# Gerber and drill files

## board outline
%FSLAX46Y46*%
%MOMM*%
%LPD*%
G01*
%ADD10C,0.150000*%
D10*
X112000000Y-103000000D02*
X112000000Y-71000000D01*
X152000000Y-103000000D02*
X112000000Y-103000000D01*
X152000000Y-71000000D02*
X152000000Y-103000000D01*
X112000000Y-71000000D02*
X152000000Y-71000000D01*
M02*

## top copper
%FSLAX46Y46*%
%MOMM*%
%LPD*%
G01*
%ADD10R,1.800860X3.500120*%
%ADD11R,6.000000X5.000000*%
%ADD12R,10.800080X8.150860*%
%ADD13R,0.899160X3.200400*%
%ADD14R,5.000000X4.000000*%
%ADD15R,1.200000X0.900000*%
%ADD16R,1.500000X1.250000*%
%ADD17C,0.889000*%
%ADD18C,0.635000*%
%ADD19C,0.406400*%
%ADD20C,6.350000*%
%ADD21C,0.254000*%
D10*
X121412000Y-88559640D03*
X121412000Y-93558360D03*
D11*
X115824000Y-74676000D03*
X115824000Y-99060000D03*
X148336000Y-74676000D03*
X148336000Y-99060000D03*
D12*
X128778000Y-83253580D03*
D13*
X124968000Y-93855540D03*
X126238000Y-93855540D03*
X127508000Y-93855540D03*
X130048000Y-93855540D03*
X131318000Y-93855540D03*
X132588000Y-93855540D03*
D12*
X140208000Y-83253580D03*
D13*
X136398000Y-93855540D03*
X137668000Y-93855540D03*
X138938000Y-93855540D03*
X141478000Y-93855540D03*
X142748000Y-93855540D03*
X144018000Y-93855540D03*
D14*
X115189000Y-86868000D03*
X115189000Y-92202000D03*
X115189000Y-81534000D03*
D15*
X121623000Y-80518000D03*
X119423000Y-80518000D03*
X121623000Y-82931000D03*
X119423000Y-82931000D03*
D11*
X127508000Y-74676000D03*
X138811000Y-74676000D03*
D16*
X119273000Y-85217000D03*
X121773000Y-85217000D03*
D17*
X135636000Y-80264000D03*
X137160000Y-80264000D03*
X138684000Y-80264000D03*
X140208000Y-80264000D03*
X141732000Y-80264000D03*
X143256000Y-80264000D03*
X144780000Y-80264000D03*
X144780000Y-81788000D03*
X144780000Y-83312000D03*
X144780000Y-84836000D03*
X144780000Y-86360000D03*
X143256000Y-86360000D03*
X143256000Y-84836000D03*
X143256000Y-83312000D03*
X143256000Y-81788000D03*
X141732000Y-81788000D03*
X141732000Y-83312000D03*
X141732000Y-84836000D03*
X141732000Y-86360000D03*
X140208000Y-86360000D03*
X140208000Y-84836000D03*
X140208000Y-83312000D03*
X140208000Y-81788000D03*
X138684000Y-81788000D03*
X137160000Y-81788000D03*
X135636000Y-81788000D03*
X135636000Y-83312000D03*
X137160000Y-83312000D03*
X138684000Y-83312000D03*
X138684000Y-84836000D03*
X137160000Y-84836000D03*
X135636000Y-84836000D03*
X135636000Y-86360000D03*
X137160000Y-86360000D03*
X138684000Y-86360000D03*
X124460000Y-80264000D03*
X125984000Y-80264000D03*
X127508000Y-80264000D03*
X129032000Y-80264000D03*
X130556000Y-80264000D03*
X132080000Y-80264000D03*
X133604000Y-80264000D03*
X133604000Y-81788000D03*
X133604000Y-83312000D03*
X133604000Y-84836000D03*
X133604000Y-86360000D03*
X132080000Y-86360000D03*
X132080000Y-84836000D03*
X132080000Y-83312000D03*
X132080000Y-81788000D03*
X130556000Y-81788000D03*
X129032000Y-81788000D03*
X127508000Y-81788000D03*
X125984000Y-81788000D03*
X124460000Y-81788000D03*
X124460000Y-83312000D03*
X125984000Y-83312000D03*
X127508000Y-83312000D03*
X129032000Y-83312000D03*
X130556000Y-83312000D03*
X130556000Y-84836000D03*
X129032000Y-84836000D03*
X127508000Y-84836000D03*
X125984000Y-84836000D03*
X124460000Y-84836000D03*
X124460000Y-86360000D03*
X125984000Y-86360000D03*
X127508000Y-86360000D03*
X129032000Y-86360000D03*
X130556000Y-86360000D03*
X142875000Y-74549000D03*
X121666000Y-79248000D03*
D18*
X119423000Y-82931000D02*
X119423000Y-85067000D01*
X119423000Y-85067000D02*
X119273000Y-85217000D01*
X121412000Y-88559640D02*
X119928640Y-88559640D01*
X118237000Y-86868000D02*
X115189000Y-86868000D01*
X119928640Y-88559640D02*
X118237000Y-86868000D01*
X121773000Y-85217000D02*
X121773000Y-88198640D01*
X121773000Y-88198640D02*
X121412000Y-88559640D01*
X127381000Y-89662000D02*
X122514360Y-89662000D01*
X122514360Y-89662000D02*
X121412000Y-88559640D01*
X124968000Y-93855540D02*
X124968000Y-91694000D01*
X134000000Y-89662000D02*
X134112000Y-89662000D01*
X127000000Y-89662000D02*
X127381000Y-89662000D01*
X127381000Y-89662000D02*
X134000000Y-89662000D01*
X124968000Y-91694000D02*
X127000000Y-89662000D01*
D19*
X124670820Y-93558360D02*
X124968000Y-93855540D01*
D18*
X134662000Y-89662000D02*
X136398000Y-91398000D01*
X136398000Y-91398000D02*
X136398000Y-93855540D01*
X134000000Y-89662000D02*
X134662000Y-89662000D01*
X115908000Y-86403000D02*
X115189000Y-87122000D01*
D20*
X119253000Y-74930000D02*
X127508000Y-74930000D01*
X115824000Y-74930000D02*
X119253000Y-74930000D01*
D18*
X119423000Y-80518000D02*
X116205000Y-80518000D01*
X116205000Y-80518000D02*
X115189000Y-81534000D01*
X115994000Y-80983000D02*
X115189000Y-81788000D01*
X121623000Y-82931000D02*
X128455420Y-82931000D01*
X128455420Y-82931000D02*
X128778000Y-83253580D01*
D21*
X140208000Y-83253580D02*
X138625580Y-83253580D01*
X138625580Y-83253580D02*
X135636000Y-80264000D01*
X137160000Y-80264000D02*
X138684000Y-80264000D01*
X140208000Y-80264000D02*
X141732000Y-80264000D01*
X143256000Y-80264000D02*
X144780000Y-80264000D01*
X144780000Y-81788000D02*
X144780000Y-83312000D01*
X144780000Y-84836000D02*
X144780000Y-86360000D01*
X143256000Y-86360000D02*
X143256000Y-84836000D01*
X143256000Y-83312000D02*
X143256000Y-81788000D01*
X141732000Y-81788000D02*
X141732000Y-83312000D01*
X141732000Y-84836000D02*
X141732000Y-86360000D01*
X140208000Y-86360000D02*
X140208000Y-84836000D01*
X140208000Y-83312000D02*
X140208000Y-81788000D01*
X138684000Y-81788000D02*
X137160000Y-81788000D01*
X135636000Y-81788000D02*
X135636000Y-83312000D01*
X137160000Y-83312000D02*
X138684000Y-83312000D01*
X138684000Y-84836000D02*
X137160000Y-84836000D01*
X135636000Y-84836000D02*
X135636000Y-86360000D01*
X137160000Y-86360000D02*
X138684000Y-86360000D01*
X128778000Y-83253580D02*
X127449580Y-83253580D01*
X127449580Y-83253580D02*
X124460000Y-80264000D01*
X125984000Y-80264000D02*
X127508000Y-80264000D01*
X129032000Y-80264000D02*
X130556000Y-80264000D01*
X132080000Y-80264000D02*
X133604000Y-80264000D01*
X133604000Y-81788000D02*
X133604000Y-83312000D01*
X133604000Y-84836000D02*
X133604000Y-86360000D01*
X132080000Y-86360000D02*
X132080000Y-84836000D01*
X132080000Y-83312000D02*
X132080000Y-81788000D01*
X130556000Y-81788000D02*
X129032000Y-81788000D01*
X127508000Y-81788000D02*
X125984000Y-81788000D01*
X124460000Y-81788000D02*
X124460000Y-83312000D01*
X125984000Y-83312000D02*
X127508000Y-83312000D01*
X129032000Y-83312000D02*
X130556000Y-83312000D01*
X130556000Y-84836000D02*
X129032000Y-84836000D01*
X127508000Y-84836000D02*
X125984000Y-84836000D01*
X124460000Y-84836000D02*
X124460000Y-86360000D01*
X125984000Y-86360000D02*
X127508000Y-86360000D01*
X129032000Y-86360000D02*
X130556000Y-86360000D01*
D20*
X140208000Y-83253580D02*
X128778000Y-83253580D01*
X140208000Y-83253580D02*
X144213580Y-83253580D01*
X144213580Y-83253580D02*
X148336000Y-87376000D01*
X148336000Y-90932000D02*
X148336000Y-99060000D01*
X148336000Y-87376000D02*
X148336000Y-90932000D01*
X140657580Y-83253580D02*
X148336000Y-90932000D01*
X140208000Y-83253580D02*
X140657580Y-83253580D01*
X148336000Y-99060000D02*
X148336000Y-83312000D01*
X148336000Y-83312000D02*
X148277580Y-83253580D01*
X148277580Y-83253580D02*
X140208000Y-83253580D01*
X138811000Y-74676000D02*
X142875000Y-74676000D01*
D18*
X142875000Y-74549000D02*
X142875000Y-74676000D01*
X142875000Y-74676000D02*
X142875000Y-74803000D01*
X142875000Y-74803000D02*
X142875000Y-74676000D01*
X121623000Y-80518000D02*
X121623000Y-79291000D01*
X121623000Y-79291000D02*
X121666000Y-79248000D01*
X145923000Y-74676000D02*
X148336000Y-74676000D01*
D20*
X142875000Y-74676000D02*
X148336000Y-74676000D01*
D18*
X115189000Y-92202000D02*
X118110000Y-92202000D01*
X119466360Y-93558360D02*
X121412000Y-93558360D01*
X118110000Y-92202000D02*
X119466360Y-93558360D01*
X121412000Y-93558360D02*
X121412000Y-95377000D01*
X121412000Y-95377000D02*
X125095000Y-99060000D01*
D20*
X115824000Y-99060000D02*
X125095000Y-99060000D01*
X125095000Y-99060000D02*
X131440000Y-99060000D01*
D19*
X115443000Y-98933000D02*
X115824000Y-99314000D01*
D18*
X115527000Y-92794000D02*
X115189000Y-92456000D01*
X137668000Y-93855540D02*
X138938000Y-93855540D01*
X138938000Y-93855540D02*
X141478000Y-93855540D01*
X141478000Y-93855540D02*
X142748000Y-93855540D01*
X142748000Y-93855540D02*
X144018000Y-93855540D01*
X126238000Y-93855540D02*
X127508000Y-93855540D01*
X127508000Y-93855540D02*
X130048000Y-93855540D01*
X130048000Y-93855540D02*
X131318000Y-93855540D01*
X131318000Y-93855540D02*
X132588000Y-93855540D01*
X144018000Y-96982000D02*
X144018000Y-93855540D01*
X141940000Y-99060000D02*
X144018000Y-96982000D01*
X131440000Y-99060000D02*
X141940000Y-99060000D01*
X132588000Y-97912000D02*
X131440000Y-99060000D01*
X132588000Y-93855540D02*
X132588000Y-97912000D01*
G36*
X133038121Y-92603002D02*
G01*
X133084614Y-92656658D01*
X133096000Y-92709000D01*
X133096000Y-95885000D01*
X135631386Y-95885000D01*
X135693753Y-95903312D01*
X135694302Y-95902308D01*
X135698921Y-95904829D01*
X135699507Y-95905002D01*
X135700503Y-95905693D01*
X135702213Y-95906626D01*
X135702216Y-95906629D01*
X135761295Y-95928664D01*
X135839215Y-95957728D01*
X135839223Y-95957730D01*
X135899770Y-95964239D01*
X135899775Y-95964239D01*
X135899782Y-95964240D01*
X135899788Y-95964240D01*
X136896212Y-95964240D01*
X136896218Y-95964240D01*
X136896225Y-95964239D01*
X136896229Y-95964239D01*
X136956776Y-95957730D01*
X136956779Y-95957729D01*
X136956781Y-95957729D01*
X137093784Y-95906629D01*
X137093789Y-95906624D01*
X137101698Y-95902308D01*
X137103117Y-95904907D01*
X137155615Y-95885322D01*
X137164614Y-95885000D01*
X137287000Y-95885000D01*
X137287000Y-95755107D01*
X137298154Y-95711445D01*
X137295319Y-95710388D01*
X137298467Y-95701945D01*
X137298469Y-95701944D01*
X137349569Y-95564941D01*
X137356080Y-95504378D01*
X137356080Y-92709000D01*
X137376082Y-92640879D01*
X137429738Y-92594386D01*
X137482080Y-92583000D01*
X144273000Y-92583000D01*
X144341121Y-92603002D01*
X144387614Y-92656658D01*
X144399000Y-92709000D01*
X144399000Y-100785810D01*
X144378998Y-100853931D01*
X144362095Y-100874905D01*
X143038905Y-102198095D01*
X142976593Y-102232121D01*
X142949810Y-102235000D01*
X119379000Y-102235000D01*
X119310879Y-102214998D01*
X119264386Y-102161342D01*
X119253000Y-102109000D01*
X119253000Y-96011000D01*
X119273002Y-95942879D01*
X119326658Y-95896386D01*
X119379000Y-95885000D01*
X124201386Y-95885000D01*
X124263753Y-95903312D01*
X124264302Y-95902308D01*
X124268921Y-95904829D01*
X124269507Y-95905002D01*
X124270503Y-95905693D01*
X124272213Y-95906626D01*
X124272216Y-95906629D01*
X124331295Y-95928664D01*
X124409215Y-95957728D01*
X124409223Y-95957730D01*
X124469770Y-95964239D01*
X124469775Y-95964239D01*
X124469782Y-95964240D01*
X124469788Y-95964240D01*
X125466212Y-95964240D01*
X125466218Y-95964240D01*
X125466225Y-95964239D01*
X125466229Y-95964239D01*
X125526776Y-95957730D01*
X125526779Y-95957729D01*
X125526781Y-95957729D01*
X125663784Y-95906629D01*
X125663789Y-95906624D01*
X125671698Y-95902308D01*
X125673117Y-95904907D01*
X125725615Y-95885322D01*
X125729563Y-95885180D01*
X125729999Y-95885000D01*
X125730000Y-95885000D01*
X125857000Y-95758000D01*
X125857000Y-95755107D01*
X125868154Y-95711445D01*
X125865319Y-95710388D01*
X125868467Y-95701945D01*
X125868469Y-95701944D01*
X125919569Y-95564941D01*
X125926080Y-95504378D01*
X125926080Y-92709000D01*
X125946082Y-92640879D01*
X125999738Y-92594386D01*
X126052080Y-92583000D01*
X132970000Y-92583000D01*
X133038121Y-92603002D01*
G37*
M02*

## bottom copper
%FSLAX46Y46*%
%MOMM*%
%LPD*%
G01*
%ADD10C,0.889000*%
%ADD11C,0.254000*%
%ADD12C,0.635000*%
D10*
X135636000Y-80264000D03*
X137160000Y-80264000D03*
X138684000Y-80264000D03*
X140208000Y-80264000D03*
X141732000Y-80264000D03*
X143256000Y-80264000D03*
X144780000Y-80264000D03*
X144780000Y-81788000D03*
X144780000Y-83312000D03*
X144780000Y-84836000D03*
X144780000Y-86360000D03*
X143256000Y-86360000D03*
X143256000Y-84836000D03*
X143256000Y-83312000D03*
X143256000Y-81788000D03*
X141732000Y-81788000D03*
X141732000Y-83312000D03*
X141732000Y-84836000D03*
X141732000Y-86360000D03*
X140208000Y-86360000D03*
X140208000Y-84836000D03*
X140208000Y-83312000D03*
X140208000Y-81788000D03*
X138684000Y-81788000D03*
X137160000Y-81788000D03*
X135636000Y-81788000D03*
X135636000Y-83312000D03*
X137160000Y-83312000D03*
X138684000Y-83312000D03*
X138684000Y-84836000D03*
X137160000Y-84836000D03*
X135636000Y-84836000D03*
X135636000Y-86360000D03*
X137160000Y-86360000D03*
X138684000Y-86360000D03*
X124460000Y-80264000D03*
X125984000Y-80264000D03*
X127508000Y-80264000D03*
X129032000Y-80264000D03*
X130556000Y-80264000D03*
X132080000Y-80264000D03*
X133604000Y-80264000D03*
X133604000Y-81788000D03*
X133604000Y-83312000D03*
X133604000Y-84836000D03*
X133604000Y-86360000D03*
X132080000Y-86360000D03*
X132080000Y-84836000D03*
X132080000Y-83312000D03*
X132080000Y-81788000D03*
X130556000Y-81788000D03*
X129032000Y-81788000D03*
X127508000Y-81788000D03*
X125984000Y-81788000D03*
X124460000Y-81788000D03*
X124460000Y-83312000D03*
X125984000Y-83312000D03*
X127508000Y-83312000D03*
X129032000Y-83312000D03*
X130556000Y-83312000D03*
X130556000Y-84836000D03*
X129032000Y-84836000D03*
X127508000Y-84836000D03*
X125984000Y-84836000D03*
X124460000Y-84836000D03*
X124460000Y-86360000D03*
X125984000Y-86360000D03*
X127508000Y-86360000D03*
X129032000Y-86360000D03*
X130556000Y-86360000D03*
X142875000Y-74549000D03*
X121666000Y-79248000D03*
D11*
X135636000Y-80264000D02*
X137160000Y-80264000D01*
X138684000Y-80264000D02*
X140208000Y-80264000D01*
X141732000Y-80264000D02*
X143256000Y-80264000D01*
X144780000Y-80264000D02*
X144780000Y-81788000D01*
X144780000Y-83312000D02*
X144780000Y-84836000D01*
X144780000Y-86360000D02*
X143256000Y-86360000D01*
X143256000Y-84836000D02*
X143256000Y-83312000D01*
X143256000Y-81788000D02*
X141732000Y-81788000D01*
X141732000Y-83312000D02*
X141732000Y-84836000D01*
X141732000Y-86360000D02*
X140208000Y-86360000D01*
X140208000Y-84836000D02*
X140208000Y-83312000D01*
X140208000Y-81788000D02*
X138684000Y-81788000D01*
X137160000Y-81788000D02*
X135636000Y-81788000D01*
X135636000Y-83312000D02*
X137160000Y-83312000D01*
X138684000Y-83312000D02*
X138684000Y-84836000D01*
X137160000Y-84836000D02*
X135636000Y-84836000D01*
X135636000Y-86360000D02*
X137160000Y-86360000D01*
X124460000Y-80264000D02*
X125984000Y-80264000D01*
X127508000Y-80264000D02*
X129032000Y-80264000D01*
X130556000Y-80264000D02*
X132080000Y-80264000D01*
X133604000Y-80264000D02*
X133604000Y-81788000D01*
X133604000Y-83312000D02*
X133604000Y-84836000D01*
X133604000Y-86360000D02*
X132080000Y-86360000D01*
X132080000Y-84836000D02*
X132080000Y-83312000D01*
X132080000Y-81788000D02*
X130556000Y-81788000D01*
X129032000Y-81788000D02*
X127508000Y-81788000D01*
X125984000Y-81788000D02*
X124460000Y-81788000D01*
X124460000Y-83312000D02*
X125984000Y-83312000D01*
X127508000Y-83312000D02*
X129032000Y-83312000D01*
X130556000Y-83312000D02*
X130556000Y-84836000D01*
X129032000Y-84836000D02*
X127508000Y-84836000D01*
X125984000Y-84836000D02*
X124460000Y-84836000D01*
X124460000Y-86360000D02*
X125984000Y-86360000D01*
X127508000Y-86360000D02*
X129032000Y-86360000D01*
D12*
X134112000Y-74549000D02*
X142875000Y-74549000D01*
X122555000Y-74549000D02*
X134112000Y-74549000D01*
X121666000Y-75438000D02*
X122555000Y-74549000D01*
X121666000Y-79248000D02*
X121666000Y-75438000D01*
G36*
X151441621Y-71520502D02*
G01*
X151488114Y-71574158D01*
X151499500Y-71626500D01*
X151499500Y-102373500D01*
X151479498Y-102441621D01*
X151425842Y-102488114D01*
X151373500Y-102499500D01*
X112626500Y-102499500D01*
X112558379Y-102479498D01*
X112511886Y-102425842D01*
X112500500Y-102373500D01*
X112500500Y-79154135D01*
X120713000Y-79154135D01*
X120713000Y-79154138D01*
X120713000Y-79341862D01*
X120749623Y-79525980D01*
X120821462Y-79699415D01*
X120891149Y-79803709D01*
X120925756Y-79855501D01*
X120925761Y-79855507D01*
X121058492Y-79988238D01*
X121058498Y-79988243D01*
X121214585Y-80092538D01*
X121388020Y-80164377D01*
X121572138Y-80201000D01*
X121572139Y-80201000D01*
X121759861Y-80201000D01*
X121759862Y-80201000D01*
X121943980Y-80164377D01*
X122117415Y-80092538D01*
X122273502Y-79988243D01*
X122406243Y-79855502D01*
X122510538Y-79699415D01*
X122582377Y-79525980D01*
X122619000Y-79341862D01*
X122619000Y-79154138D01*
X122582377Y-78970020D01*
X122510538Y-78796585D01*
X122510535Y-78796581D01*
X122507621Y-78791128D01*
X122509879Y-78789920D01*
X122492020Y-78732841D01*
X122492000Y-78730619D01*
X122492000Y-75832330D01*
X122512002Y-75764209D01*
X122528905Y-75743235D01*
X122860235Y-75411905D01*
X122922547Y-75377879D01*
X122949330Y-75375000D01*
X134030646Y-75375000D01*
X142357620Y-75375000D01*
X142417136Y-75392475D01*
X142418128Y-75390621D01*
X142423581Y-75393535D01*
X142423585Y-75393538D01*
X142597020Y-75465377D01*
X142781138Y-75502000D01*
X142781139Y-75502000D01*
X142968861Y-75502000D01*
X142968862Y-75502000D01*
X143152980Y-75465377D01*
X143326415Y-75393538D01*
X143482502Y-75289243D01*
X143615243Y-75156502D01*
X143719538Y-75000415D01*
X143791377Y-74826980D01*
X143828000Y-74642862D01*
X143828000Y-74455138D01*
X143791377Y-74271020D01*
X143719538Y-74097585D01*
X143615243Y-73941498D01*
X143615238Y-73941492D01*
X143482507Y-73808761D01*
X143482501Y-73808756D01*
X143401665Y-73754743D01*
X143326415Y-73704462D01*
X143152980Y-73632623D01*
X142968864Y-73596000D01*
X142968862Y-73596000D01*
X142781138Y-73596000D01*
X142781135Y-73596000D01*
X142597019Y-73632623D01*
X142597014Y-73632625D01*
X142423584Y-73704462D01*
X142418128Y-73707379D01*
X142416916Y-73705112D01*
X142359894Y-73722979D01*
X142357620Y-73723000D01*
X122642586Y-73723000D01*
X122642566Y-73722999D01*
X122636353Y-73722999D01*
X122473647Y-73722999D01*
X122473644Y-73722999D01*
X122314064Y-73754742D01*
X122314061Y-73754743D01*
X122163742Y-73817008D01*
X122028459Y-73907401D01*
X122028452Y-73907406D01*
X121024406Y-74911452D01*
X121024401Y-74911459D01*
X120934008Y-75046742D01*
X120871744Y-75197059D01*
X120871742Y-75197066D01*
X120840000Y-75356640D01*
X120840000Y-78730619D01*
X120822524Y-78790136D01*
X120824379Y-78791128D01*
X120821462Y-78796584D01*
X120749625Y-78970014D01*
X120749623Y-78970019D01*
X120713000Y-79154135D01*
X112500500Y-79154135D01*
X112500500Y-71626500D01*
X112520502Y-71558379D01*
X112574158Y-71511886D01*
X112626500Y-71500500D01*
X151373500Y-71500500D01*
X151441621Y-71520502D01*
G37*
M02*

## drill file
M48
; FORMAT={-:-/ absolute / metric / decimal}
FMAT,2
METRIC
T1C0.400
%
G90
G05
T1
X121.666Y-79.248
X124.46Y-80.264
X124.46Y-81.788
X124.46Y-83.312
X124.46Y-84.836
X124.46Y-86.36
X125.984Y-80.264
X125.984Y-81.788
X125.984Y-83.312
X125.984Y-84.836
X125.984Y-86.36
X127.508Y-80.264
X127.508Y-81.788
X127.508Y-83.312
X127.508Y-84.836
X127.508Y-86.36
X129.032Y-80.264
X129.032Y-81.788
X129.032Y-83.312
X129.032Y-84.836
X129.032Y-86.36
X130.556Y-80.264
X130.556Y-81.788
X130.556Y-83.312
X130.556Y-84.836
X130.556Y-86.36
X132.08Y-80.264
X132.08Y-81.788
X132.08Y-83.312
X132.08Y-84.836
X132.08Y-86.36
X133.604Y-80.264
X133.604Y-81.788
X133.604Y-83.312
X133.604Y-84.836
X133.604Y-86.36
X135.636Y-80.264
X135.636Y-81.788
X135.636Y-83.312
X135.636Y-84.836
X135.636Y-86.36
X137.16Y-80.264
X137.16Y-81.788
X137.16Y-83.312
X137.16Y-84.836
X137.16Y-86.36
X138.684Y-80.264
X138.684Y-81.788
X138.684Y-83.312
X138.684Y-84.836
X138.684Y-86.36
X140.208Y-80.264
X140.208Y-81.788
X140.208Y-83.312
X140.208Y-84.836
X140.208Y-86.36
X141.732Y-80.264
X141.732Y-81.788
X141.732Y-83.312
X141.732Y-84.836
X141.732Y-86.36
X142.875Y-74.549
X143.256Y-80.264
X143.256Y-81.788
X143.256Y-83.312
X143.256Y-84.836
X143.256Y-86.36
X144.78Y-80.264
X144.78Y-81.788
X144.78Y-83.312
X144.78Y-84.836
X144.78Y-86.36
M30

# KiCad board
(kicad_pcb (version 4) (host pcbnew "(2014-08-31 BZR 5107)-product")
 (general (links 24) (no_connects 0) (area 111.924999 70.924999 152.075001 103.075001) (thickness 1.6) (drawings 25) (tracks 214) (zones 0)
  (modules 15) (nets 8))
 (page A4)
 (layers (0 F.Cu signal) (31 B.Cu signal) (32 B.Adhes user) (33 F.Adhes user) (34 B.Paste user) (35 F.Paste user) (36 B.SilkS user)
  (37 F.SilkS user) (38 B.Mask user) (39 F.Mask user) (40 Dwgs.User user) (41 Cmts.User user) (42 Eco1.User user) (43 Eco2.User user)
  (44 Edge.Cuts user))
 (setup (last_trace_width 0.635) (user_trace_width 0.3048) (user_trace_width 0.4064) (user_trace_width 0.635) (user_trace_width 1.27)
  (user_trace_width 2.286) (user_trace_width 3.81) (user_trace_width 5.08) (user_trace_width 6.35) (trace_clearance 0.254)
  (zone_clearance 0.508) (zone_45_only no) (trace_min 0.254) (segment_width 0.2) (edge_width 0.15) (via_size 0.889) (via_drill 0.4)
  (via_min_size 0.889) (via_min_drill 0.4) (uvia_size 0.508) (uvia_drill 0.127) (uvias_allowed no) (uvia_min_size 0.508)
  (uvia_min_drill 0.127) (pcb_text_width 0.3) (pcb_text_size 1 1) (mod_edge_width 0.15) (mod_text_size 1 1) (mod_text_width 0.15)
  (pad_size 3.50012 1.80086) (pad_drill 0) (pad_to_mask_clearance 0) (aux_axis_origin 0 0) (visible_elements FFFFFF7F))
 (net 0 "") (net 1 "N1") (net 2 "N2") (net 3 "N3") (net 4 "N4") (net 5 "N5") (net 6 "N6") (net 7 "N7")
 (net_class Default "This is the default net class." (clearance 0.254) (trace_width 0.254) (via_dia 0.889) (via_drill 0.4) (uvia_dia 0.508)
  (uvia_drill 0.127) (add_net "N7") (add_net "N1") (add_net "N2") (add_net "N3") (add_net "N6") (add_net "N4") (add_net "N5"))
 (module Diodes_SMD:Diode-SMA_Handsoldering (layer F.Cu) (at 121.412 91.059 270)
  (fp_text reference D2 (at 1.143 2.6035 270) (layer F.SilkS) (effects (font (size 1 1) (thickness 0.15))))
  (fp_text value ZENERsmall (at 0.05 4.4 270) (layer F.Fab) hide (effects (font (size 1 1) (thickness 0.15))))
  (pad 2 smd rect (at -2.49936 0 270) (size 3.50012 1.80086) (layers F.Cu F.Paste F.Mask) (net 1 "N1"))
  (pad 1 smd rect (at 2.49936 0 270) (size 3.50012 1.80086) (layers F.Cu F.Paste F.Mask) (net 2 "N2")))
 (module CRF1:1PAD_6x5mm (layer F.Cu) (at 115.824 74.676)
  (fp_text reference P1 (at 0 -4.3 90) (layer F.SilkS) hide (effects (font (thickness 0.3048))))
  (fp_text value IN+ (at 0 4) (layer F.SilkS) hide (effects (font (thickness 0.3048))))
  (pad 1 smd rect (at 0 0) (size 6 5) (layers F.Cu F.Paste F.Mask) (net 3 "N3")))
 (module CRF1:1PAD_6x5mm (layer F.Cu) (at 115.824 99.06)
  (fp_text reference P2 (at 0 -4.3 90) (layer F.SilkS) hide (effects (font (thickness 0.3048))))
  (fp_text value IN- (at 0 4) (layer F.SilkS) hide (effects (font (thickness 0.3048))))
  (pad 1 smd rect (at 0 0) (size 6 5) (layers F.Cu F.Paste F.Mask) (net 2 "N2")))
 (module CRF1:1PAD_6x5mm (layer F.Cu) (at 148.336 74.676)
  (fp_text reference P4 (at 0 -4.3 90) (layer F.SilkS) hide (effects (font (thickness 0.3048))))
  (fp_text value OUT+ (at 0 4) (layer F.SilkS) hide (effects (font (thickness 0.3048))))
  (pad 1 smd rect (at 0 0) (size 6 5) (layers F.Cu F.Paste F.Mask) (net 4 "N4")))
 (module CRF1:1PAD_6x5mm (layer F.Cu) (at 148.336 99.06)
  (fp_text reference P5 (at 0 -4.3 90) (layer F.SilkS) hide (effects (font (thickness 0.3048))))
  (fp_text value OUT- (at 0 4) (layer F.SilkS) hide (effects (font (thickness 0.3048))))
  (pad 1 smd rect (at 0 0) (size 6 5) (layers F.Cu F.Paste F.Mask) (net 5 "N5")))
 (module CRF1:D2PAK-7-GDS (layer F.Cu) (at 128.778 89.154)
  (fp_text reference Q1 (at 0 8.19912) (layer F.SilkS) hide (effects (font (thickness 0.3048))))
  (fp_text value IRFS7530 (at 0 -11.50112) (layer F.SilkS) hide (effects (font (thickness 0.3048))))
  (pad D smd rect (at 0 -5.90042) (size 10.80008 8.15086) (layers F.Cu F.Paste F.Mask) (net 5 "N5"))
  (pad G smd rect (at -3.81 4.70154) (size 0.89916 3.2004) (layers F.Cu F.Paste F.Mask) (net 1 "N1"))
  (pad S smd rect (at -2.54 4.70154) (size 0.89916 3.2004) (layers F.Cu F.Paste F.Mask) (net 2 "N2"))
  (pad S smd rect (at -1.27 4.70154) (size 0.89916 3.2004) (layers F.Cu F.Paste F.Mask) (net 2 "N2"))
  (pad S smd rect (at 1.27 4.70154) (size 0.89916 3.2004) (layers F.Cu F.Paste F.Mask) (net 2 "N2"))
  (pad S smd rect (at 2.54 4.70154) (size 0.89916 3.2004) (layers F.Cu F.Paste F.Mask) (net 2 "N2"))
  (pad S smd rect (at 3.81 4.70154) (size 0.89916 3.2004) (layers F.Cu F.Paste F.Mask) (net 2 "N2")))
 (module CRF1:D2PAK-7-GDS (layer F.Cu) (at 140.208 89.154)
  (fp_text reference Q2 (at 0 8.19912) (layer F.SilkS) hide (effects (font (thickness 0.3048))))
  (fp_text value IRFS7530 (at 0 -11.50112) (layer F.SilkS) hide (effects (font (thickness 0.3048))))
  (pad D smd rect (at 0 -5.90042) (size 10.80008 8.15086) (layers F.Cu F.Paste F.Mask) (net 5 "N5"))
  (pad G smd rect (at -3.81 4.70154) (size 0.89916 3.2004) (layers F.Cu F.Paste F.Mask) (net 1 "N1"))
  (pad S smd rect (at -2.54 4.70154) (size 0.89916 3.2004) (layers F.Cu F.Paste F.Mask) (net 2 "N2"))
  (pad S smd rect (at -1.27 4.70154) (size 0.89916 3.2004) (layers F.Cu F.Paste F.Mask) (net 2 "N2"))
  (pad S smd rect (at 1.27 4.70154) (size 0.89916 3.2004) (layers F.Cu F.Paste F.Mask) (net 2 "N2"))
  (pad S smd rect (at 2.54 4.70154) (size 0.89916 3.2004) (layers F.Cu F.Paste F.Mask) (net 2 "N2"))
  (pad S smd rect (at 3.81 4.70154) (size 0.89916 3.2004) (layers F.Cu F.Paste F.Mask) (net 2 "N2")))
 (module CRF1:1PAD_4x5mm (layer F.Cu) (at 115.189 86.868 90)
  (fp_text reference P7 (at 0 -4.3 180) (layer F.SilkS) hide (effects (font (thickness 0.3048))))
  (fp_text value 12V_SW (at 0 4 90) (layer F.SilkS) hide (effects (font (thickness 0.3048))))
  (pad 1 smd rect (at 0 0 90) (size 4 5) (layers F.Cu F.Paste F.Mask) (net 1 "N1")))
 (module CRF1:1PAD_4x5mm (layer F.Cu) (at 115.189 92.202 90)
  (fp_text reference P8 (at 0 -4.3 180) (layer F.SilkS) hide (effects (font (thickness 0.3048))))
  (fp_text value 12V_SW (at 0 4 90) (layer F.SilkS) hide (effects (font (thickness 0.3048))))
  (pad 1 smd rect (at 0 0 90) (size 4 5) (layers F.Cu F.Paste F.Mask) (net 2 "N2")))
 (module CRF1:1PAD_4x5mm (layer F.Cu) (at 115.189 81.534 90)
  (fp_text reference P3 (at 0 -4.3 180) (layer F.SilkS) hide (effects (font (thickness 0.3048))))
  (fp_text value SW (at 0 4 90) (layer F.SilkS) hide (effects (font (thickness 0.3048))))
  (pad 1 smd rect (at 0 0 90) (size 4 5) (layers F.Cu F.Paste F.Mask) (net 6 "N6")))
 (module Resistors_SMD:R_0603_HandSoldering (layer F.Cu) (at 120.523 80.518 180)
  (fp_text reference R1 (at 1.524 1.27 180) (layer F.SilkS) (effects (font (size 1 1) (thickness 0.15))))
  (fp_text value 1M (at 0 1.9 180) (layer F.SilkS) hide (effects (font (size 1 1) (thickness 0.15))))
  (pad 1 smd rect (at -1.1 0 180) (size 1.2 0.9) (layers F.Cu F.Paste F.Mask) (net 4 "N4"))
  (pad 2 smd rect (at 1.1 0 180) (size 1.2 0.9) (layers F.Cu F.Paste F.Mask) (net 6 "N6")))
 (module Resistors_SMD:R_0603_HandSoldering (layer F.Cu) (at 120.523 82.931 180)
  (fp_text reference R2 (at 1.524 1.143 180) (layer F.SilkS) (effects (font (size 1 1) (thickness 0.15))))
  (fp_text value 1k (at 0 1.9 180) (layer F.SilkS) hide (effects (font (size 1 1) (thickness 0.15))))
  (pad 1 smd rect (at -1.1 0 180) (size 1.2 0.9) (layers F.Cu F.Paste F.Mask) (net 5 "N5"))
  (pad 2 smd rect (at 1.1 0 180) (size 1.2 0.9) (layers F.Cu F.Paste F.Mask) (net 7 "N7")))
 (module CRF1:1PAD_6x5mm (layer F.Cu) (at 127.508 74.676)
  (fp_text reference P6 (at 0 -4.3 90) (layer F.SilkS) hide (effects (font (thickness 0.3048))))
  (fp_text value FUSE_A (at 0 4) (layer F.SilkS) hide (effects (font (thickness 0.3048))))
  (pad 1 smd rect (at 0 0) (size 6 5) (layers F.Cu F.Paste F.Mask) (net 3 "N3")))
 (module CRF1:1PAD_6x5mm (layer F.Cu) (at 138.811 74.676)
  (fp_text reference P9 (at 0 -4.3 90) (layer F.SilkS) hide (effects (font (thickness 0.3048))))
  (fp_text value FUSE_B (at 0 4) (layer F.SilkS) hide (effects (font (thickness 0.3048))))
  (pad 1 smd rect (at 0 0) (size 6 5) (layers F.Cu F.Paste F.Mask) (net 4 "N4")))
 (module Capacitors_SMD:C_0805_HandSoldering (layer F.Cu) (at 120.523 85.217)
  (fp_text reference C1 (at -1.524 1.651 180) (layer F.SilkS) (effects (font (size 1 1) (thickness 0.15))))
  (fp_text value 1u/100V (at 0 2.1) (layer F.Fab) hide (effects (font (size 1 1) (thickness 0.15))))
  (pad 1 smd rect (at -1.25 0) (size 1.5 1.25) (layers F.Cu F.Paste F.Mask) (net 7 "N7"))
  (pad 2 smd rect (at 1.25 0) (size 1.5 1.25) (layers F.Cu F.Paste F.Mask) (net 1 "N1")))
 (gr_line (start 112 103) (end 112 71) (angle 90) (layer Edge.Cuts) (width 0.15))
 (gr_line (start 152 103) (end 112 103) (angle 90) (layer Edge.Cuts) (width 0.15))
 (gr_line (start 152 71) (end 152 103) (angle 90) (layer Edge.Cuts) (width 0.15))
 (gr_line (start 112 71) (end 152 71) (angle 90) (layer Edge.Cuts) (width 0.15))
 (segment (start 119.423 82.931) (end 119.423 85.067) (width 0.635) (layer F.Cu) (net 7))
 (segment (start 119.423 85.067) (end 119.273 85.217) (width 0.635) (layer F.Cu) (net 7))
 (segment (start 121.412 88.55964) (end 119.92864 88.55964) (width 0.635) (layer F.Cu) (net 1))
 (segment (start 118.237 86.868) (end 115.189 86.868) (width 0.635) (layer F.Cu) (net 1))
 (segment (start 119.92864 88.55964) (end 118.237 86.868) (width 0.635) (layer F.Cu) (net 1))
 (segment (start 121.773 85.217) (end 121.773 88.19864) (width 0.635) (layer F.Cu) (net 1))
 (segment (start 121.773 88.19864) (end 121.412 88.55964) (width 0.635) (layer F.Cu) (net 1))
 (segment (start 127.381 89.662) (end 122.51436 89.662) (width 0.635) (layer F.Cu) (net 1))
 (segment (start 122.51436 89.662) (end 121.412 88.55964) (width 0.635) (layer F.Cu) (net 1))
 (segment (start 124.968 93.85554) (end 124.968 91.694) (width 0.635) (layer F.Cu) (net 1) (status 10))
 (segment (start 134 89.662) (end 134.112 89.662) (width 0.635) (layer F.Cu) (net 1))
 (segment (start 127 89.662) (end 127.381 89.662) (width 0.635) (layer F.Cu) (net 1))
 (segment (start 127.381 89.662) (end 134 89.662) (width 0.635) (layer F.Cu) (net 1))
 (segment (start 124.968 91.694) (end 127 89.662) (width 0.635) (layer F.Cu) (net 1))
 (segment (start 124.67082 93.55836) (end 124.968 93.85554) (width 0.4064) (layer F.Cu) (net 1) (status 30))
 (segment (start 134.662 89.662) (end 136.398 91.398) (width 0.635) (layer F.Cu) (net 1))
 (segment (start 136.398 91.398) (end 136.398 93.85554) (width 0.635) (layer F.Cu) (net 1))
 (segment (start 134 89.662) (end 134.662 89.662) (width 0.635) (layer F.Cu) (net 1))
 (segment (start 115.908 86.403) (end 115.189 87.122) (width 0.635) (layer F.Cu) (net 1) (status 30))
 (segment (start 119.253 74.93) (end 127.508 74.93) (width 6.35) (layer F.Cu) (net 3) (status 30))
 (segment (start 115.824 74.93) (end 119.253 74.93) (width 6.35) (layer F.Cu) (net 3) (status 30))
 (segment (start 119.423 80.518) (end 116.205 80.518) (width 0.635) (layer F.Cu) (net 6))
 (segment (start 116.205 80.518) (end 115.189 81.534) (width 0.635) (layer F.Cu) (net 6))
 (segment (start 115.994 80.983) (end 115.189 81.788) (width 0.635) (layer F.Cu) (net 6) (status 30))
 (segment (start 121.623 82.931) (end 128.45542 82.931) (width 0.635) (layer F.Cu) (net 5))
 (segment (start 128.45542 82.931) (end 128.778 83.25358) (width 0.635) (layer F.Cu) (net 5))
 (segment (start 140.208 83.25358) (end 138.62558 83.25358) (width 0.254) (layer F.Cu) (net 5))
 (segment (start 138.62558 83.25358) (end 135.636 80.264) (width 0.254) (layer F.Cu) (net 5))
 (via (at 135.636 80.264) (size 0.889) (layers F.Cu B.Cu) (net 5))
 (segment (start 135.636 80.264) (end 137.16 80.264) (width 0.254) (layer B.Cu) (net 5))
 (via (at 137.16 80.264) (size 0.889) (layers F.Cu B.Cu) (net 5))
 (segment (start 137.16 80.264) (end 138.684 80.264) (width 0.254) (layer F.Cu) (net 5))
 (via (at 138.684 80.264) (size 0.889) (layers F.Cu B.Cu) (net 5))
 (segment (start 138.684 80.264) (end 140.208 80.264) (width 0.254) (layer B.Cu) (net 5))
 (via (at 140.208 80.264) (size 0.889) (layers F.Cu B.Cu) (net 5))
 (segment (start 140.208 80.264) (end 141.732 80.264) (width 0.254) (layer F.Cu) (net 5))
 (via (at 141.732 80.264) (size 0.889) (layers F.Cu B.Cu) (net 5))
 (segment (start 141.732 80.264) (end 143.256 80.264) (width 0.254) (layer B.Cu) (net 5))
 (via (at 143.256 80.264) (size 0.889) (layers F.Cu B.Cu) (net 5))
 (segment (start 143.256 80.264) (end 144.78 80.264) (width 0.254) (layer F.Cu) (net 5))
 (via (at 144.78 80.264) (size 0.889) (layers F.Cu B.Cu) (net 5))
 (segment (start 144.78 80.264) (end 144.78 81.788) (width 0.254) (layer B.Cu) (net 5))
 (via (at 144.78 81.788) (size 0.889) (layers F.Cu B.Cu) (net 5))
 (segment (start 144.78 81.788) (end 144.78 83.312) (width 0.254) (layer F.Cu) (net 5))
 (via (at 144.78 83.312) (size 0.889) (layers F.Cu B.Cu) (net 5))
 (segment (start 144.78 83.312) (end 144.78 84.836) (width 0.254) (layer B.Cu) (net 5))
 (via (at 144.78 84.836) (size 0.889) (layers F.Cu B.Cu) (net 5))
 (segment (start 144.78 84.836) (end 144.78 86.36) (width 0.254) (layer F.Cu) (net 5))
 (via (at 144.78 86.36) (size 0.889) (layers F.Cu B.Cu) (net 5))
 (segment (start 144.78 86.36) (end 143.256 86.36) (width 0.254) (layer B.Cu) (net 5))
 (via (at 143.256 86.36) (size 0.889) (layers F.Cu B.Cu) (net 5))
 (segment (start 143.256 86.36) (end 143.256 84.836) (width 0.254) (layer F.Cu) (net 5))
 (via (at 143.256 84.836) (size 0.889) (layers F.Cu B.Cu) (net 5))
 (segment (start 143.256 84.836) (end 143.256 83.312) (width 0.254) (layer B.Cu) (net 5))
 (via (at 143.256 83.312) (size 0.889) (layers F.Cu B.Cu) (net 5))
 (segment (start 143.256 83.312) (end 143.256 81.788) (width 0.254) (layer F.Cu) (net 5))
 (via (at 143.256 81.788) (size 0.889) (layers F.Cu B.Cu) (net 5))
 (segment (start 143.256 81.788) (end 141.732 81.788) (width 0.254) (layer B.Cu) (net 5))
 (via (at 141.732 81.788) (size 0.889) (layers F.Cu B.Cu) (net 5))
 (segment (start 141.732 81.788) (end 141.732 83.312) (width 0.254) (layer F.Cu) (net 5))
 (via (at 141.732 83.312) (size 0.889) (layers F.Cu B.Cu) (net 5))
 (segment (start 141.732 83.312) (end 141.732 84.836) (width 0.254) (layer B.Cu) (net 5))
 (via (at 141.732 84.836) (size 0.889) (layers F.Cu B.Cu) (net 5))
 (segment (start 141.732 84.836) (end 141.732 86.36) (width 0.254) (layer F.Cu) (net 5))
 (via (at 141.732 86.36) (size 0.889) (layers F.Cu B.Cu) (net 5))
 (segment (start 141.732 86.36) (end 140.208 86.36) (width 0.254) (layer B.Cu) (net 5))
 (via (at 140.208 86.36) (size 0.889) (layers F.Cu B.Cu) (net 5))
 (segment (start 140.208 86.36) (end 140.208 84.836) (width 0.254) (layer F.Cu) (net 5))
 (via (at 140.208 84.836) (size 0.889) (layers F.Cu B.Cu) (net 5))
 (segment (start 140.208 84.836) (end 140.208 83.312) (width 0.254) (layer B.Cu) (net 5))
 (via (at 140.208 83.312) (size 0.889) (layers F.Cu B.Cu) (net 5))
 (segment (start 140.208 83.312) (end 140.208 81.788) (width 0.254) (layer F.Cu) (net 5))
 (via (at 140.208 81.788) (size 0.889) (layers F.Cu B.Cu) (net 5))
 (segment (start 140.208 81.788) (end 138.684 81.788) (width 0.254) (layer B.Cu) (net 5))
 (via (at 138.684 81.788) (size 0.889) (layers F.Cu B.Cu) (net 5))
 (segment (start 138.684 81.788) (end 137.16 81.788) (width 0.254) (layer F.Cu) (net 5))
 (via (at 137.16 81.788) (size 0.889) (layers F.Cu B.Cu) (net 5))
 (segment (start 137.16 81.788) (end 135.636 81.788) (width 0.254) (layer B.Cu) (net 5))
 (via (at 135.636 81.788) (size 0.889) (layers F.Cu B.Cu) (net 5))
 (segment (start 135.636 81.788) (end 135.636 83.312) (width 0.254) (layer F.Cu) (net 5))
 (via (at 135.636 83.312) (size 0.889) (layers F.Cu B.Cu) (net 5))
 (segment (start 135.636 83.312) (end 137.16 83.312) (width 0.254) (layer B.Cu) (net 5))
 (via (at 137.16 83.312) (size 0.889) (layers F.Cu B.Cu) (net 5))
 (segment (start 137.16 83.312) (end 138.684 83.312) (width 0.254) (layer F.Cu) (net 5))
 (via (at 138.684 83.312) (size 0.889) (layers F.Cu B.Cu) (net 5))
 (segment (start 138.684 83.312) (end 138.684 84.836) (width 0.254) (layer B.Cu) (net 5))
 (via (at 138.684 84.836) (size 0.889) (layers F.Cu B.Cu) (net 5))
 (segment (start 138.684 84.836) (end 137.16 84.836) (width 0.254) (layer F.Cu) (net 5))
 (via (at 137.16 84.836) (size 0.889) (layers F.Cu B.Cu) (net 5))
 (segment (start 137.16 84.836) (end 135.636 84.836) (width 0.254) (layer B.Cu) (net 5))
 (via (at 135.636 84.836) (size 0.889) (layers F.Cu B.Cu) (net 5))
 (segment (start 135.636 84.836) (end 135.636 86.36) (width 0.254) (layer F.Cu) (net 5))
 (via (at 135.636 86.36) (size 0.889) (layers F.Cu B.Cu) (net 5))
 (segment (start 135.636 86.36) (end 137.16 86.36) (width 0.254) (layer B.Cu) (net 5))
 (via (at 137.16 86.36) (size 0.889) (layers F.Cu B.Cu) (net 5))
 (segment (start 137.16 86.36) (end 138.684 86.36) (width 0.254) (layer F.Cu) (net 5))
 (via (at 138.684 86.36) (size 0.889) (layers F.Cu B.Cu) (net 5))
 (segment (start 128.778 83.25358) (end 127.44958 83.25358) (width 0.254) (layer F.Cu) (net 5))
 (segment (start 127.44958 83.25358) (end 124.46 80.264) (width 0.254) (layer F.Cu) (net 5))
 (via (at 124.46 80.264) (size 0.889) (layers F.Cu B.Cu) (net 5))
 (segment (start 124.46 80.264) (end 125.984 80.264) (width 0.254) (layer B.Cu) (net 5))
 (via (at 125.984 80.264) (size 0.889) (layers F.Cu B.Cu) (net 5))
 (segment (start 125.984 80.264) (end 127.508 80.264) (width 0.254) (layer F.Cu) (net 5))
 (via (at 127.508 80.264) (size 0.889) (layers F.Cu B.Cu) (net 5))
 (segment (start 127.508 80.264) (end 129.032 80.264) (width 0.254) (layer B.Cu) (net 5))
 (via (at 129.032 80.264) (size 0.889) (layers F.Cu B.Cu) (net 5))
 (segment (start 129.032 80.264) (end 130.556 80.264) (width 0.254) (layer F.Cu) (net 5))
 (via (at 130.556 80.264) (size 0.889) (layers F.Cu B.Cu) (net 5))
 (segment (start 130.556 80.264) (end 132.08 80.264) (width 0.254) (layer B.Cu) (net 5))
 (via (at 132.08 80.264) (size 0.889) (layers F.Cu B.Cu) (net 5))
 (segment (start 132.08 80.264) (end 133.604 80.264) (width 0.254) (layer F.Cu) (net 5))
 (via (at 133.604 80.264) (size 0.889) (layers F.Cu B.Cu) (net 5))
 (segment (start 133.604 80.264) (end 133.604 81.788) (width 0.254) (layer B.Cu) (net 5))
 (via (at 133.604 81.788) (size 0.889) (layers F.Cu B.Cu) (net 5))
 (segment (start 133.604 81.788) (end 133.604 83.312) (width 0.254) (layer F.Cu) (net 5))
 (via (at 133.604 83.312) (size 0.889) (layers F.Cu B.Cu) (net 5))
 (segment (start 133.604 83.312) (end 133.604 84.836) (width 0.254) (layer B.Cu) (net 5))
 (via (at 133.604 84.836) (size 0.889) (layers F.Cu B.Cu) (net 5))
 (segment (start 133.604 84.836) (end 133.604 86.36) (width 0.254) (layer F.Cu) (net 5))
 (via (at 133.604 86.36) (size 0.889) (layers F.Cu B.Cu) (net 5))
 (segment (start 133.604 86.36) (end 132.08 86.36) (width 0.254) (layer B.Cu) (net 5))
 (via (at 132.08 86.36) (size 0.889) (layers F.Cu B.Cu) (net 5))
 (segment (start 132.08 86.36) (end 132.08 84.836) (width 0.254) (layer F.Cu) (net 5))
 (via (at 132.08 84.836) (size 0.889) (layers F.Cu B.Cu) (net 5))
 (segment (start 132.08 84.836) (end 132.08 83.312) (width 0.254) (layer B.Cu) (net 5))
 (via (at 132.08 83.312) (size 0.889) (layers F.Cu B.Cu) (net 5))
 (segment (start 132.08 83.312) (end 132.08 81.788) (width 0.254) (layer F.Cu) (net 5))
 (via (at 132.08 81.788) (size 0.889) (layers F.Cu B.Cu) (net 5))
 (segment (start 132.08 81.788) (end 130.556 81.788) (width 0.254) (layer B.Cu) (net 5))
 (via (at 130.556 81.788) (size 0.889) (layers F.Cu B.Cu) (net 5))
 (segment (start 130.556 81.788) (end 129.032 81.788) (width 0.254) (layer F.Cu) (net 5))
 (via (at 129.032 81.788) (size 0.889) (layers F.Cu B.Cu) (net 5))
 (segment (start 129.032 81.788) (end 127.508 81.788) (width 0.254) (layer B.Cu) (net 5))
 (via (at 127.508 81.788) (size 0.889) (layers F.Cu B.Cu) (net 5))
 (segment (start 127.508 81.788) (end 125.984 81.788) (width 0.254) (layer F.Cu) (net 5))
 (via (at 125.984 81.788) (size 0.889) (layers F.Cu B.Cu) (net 5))
 (segment (start 125.984 81.788) (end 124.46 81.788) (width 0.254) (layer B.Cu) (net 5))
 (via (at 124.46 81.788) (size 0.889) (layers F.Cu B.Cu) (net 5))
 (segment (start 124.46 81.788) (end 124.46 83.312) (width 0.254) (layer F.Cu) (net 5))
 (via (at 124.46 83.312) (size 0.889) (layers F.Cu B.Cu) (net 5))
 (segment (start 124.46 83.312) (end 125.984 83.312) (width 0.254) (layer B.Cu) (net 5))
 (via (at 125.984 83.312) (size 0.889) (layers F.Cu B.Cu) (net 5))
 (segment (start 125.984 83.312) (end 127.508 83.312) (width 0.254) (layer F.Cu) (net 5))
 (via (at 127.508 83.312) (size 0.889) (layers F.Cu B.Cu) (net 5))
 (segment (start 127.508 83.312) (end 129.032 83.312) (width 0.254) (layer B.Cu) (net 5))
 (via (at 129.032 83.312) (size 0.889) (layers F.Cu B.Cu) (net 5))
 (segment (start 129.032 83.312) (end 130.556 83.312) (width 0.254) (layer F.Cu) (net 5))
 (via (at 130.556 83.312) (size 0.889) (layers F.Cu B.Cu) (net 5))
 (segment (start 130.556 83.312) (end 130.556 84.836) (width 0.254) (layer B.Cu) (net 5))
 (via (at 130.556 84.836) (size 0.889) (layers F.Cu B.Cu) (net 5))
 (segment (start 130.556 84.836) (end 129.032 84.836) (width 0.254) (layer F.Cu) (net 5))
 (via (at 129.032 84.836) (size 0.889) (layers F.Cu B.Cu) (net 5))
 (segment (start 129.032 84.836) (end 127.508 84.836) (width 0.254) (layer B.Cu) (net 5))
 (via (at 127.508 84.836) (size 0.889) (layers F.Cu B.Cu) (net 5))
 (segment (start 127.508 84.836) (end 125.984 84.836) (width 0.254) (layer F.Cu) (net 5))
 (via (at 125.984 84.836) (size 0.889) (layers F.Cu B.Cu) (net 5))
 (segment (start 125.984 84.836) (end 124.46 84.836) (width 0.254) (layer B.Cu) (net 5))
 (via (at 124.46 84.836) (size 0.889) (layers F.Cu B.Cu) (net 5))
 (segment (start 124.46 84.836) (end 124.46 86.36) (width 0.254) (layer F.Cu) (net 5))
 (via (at 124.46 86.36) (size 0.889) (layers F.Cu B.Cu) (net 5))
 (segment (start 124.46 86.36) (end 125.984 86.36) (width 0.254) (layer B.Cu) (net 5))
 (via (at 125.984 86.36) (size 0.889) (layers F.Cu B.Cu) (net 5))
 (segment (start 125.984 86.36) (end 127.508 86.36) (width 0.254) (layer F.Cu) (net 5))
 (via (at 127.508 86.36) (size 0.889) (layers F.Cu B.Cu) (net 5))
 (segment (start 127.508 86.36) (end 129.032 86.36) (width 0.254) (layer B.Cu) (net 5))
 (via (at 129.032 86.36) (size 0.889) (layers F.Cu B.Cu) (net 5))
 (segment (start 129.032 86.36) (end 130.556 86.36) (width 0.254) (layer F.Cu) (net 5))
 (via (at 130.556 86.36) (size 0.889) (layers F.Cu B.Cu) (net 5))
 (segment (start 140.208 83.25358) (end 128.778 83.25358) (width 6.35) (layer F.Cu) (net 5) (status 30))
 (segment (start 140.208 83.25358) (end 144.21358 83.25358) (width 6.35) (layer F.Cu) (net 5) (status 30))
 (segment (start 144.21358 83.25358) (end 148.336 87.376) (width 6.35) (layer F.Cu) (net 5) (status 10))
 (segment (start 148.336 90.932) (end 148.336 99.06) (width 6.35) (layer F.Cu) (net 5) (status 20))
 (segment (start 148.336 87.376) (end 148.336 90.932) (width 6.35) (layer F.Cu) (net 5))
 (segment (start 140.65758 83.25358) (end 148.336 90.932) (width 6.35) (layer F.Cu) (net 5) (status 10))
 (segment (start 140.208 83.25358) (end 140.65758 83.25358) (width 6.35) (layer F.Cu) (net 5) (status 30))
 (segment (start 148.336 99.06) (end 148.336 83.312) (width 6.35) (layer F.Cu) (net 5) (status 10))
 (segment (start 148.336 83.312) (end 148.27758 83.25358) (width 6.35) (layer F.Cu) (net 5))
 (segment (start 148.27758 83.25358) (end 140.208 83.25358) (width 6.35) (layer F.Cu) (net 5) (status 20))
 (segment (start 138.811 74.676) (end 142.875 74.676) (width 6.35) (layer F.Cu) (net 4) (status 30))
 (segment (start 134.112 74.549) (end 142.875 74.549) (width 0.635) (layer B.Cu) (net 4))
 (segment (start 142.875 74.549) (end 142.875 74.676) (width 0.635) (layer F.Cu) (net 4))
 (via (at 142.875 74.549) (size 0.889) (layers F.Cu B.Cu) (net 4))
 (segment (start 142.875 74.676) (end 142.875 74.803) (width 0.635) (layer F.Cu) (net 4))
 (segment (start 142.875 74.803) (end 142.875 74.676) (width 0.635) (layer F.Cu) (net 4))
 (segment (start 121.623 80.518) (end 121.623 79.291) (width 0.635) (layer F.Cu) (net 4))
 (segment (start 122.555 74.549) (end 134.112 74.549) (width 0.635) (layer B.Cu) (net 4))
 (segment (start 121.666 75.438) (end 122.555 74.549) (width 0.635) (layer B.Cu) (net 4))
 (segment (start 121.666 79.248) (end 121.666 75.438) (width 0.635) (layer B.Cu) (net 4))
 (via (at 121.666 79.248) (size 0.889) (layers F.Cu B.Cu) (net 4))
 (segment (start 121.623 79.291) (end 121.666 79.248) (width 0.635) (layer F.Cu) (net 4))
 (segment (start 145.923 74.676) (end 148.336 74.676) (width 0.635) (layer F.Cu) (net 4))
 (segment (start 142.875 74.676) (end 148.336 74.676) (width 6.35) (layer F.Cu) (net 4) (status 30))
 (segment (start 115.189 92.202) (end 118.11 92.202) (width 0.635) (layer F.Cu) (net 2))
 (segment (start 119.46636 93.55836) (end 121.412 93.55836) (width 0.635) (layer F.Cu) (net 2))
 (segment (start 118.11 92.202) (end 119.46636 93.55836) (width 0.635) (layer F.Cu) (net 2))
 (segment (start 121.412 93.55836) (end 121.412 95.377) (width 0.635) (layer F.Cu) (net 2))
 (segment (start 121.412 95.377) (end 125.095 99.06) (width 0.635) (layer F.Cu) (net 2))
 (segment (start 115.824 99.06) (end 125.095 99.06) (width 6.35) (layer F.Cu) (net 2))
 (segment (start 125.095 99.06) (end 131.44 99.06) (width 6.35) (layer F.Cu) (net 2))
 (segment (start 115.443 98.933) (end 115.824 99.314) (width 0.4064) (layer F.Cu) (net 2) (status 30))
 (segment (start 115.527 92.794) (end 115.189 92.456) (width 0.635) (layer F.Cu) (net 2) (status 30))
 (segment (start 137.668 93.85554) (end 138.938 93.85554) (width 0.635) (layer F.Cu) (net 2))
 (segment (start 138.938 93.85554) (end 141.478 93.85554) (width 0.635) (layer F.Cu) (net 2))
 (segment (start 141.478 93.85554) (end 142.748 93.85554) (width 0.635) (layer F.Cu) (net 2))
 (segment (start 142.748 93.85554) (end 144.018 93.85554) (width 0.635) (layer F.Cu) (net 2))
 (segment (start 126.238 93.85554) (end 127.508 93.85554) (width 0.635) (layer F.Cu) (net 2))
 (segment (start 127.508 93.85554) (end 130.048 93.85554) (width 0.635) (layer F.Cu) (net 2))
 (segment (start 130.048 93.85554) (end 131.318 93.85554) (width 0.635) (layer F.Cu) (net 2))
 (segment (start 131.318 93.85554) (end 132.588 93.85554) (width 0.635) (layer F.Cu) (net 2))
 (segment (start 144.018 96.982) (end 144.018 93.85554) (width 0.635) (layer F.Cu) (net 2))
 (segment (start 141.94 99.06) (end 144.018 96.982) (width 0.635) (layer F.Cu) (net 2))
 (segment (start 131.44 99.06) (end 141.94 99.06) (width 0.635) (layer F.Cu) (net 2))
 (segment (start 132.588 97.912) (end 131.44 99.06) (width 0.635) (layer F.Cu) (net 2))
 (segment (start 132.588 93.85554) (end 132.588 97.912) (width 0.635) (layer F.Cu) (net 2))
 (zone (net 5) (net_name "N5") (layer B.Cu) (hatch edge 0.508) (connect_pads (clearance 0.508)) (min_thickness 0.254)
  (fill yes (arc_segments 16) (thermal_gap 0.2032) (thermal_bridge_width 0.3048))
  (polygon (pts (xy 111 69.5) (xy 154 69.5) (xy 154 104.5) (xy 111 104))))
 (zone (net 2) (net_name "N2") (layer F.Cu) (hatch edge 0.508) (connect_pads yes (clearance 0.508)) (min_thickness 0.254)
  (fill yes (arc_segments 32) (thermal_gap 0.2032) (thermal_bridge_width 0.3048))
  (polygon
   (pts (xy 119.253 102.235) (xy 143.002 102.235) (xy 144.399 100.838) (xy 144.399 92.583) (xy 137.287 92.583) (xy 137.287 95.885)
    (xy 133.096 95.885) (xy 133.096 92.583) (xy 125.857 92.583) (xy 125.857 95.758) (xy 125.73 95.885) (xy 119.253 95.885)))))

